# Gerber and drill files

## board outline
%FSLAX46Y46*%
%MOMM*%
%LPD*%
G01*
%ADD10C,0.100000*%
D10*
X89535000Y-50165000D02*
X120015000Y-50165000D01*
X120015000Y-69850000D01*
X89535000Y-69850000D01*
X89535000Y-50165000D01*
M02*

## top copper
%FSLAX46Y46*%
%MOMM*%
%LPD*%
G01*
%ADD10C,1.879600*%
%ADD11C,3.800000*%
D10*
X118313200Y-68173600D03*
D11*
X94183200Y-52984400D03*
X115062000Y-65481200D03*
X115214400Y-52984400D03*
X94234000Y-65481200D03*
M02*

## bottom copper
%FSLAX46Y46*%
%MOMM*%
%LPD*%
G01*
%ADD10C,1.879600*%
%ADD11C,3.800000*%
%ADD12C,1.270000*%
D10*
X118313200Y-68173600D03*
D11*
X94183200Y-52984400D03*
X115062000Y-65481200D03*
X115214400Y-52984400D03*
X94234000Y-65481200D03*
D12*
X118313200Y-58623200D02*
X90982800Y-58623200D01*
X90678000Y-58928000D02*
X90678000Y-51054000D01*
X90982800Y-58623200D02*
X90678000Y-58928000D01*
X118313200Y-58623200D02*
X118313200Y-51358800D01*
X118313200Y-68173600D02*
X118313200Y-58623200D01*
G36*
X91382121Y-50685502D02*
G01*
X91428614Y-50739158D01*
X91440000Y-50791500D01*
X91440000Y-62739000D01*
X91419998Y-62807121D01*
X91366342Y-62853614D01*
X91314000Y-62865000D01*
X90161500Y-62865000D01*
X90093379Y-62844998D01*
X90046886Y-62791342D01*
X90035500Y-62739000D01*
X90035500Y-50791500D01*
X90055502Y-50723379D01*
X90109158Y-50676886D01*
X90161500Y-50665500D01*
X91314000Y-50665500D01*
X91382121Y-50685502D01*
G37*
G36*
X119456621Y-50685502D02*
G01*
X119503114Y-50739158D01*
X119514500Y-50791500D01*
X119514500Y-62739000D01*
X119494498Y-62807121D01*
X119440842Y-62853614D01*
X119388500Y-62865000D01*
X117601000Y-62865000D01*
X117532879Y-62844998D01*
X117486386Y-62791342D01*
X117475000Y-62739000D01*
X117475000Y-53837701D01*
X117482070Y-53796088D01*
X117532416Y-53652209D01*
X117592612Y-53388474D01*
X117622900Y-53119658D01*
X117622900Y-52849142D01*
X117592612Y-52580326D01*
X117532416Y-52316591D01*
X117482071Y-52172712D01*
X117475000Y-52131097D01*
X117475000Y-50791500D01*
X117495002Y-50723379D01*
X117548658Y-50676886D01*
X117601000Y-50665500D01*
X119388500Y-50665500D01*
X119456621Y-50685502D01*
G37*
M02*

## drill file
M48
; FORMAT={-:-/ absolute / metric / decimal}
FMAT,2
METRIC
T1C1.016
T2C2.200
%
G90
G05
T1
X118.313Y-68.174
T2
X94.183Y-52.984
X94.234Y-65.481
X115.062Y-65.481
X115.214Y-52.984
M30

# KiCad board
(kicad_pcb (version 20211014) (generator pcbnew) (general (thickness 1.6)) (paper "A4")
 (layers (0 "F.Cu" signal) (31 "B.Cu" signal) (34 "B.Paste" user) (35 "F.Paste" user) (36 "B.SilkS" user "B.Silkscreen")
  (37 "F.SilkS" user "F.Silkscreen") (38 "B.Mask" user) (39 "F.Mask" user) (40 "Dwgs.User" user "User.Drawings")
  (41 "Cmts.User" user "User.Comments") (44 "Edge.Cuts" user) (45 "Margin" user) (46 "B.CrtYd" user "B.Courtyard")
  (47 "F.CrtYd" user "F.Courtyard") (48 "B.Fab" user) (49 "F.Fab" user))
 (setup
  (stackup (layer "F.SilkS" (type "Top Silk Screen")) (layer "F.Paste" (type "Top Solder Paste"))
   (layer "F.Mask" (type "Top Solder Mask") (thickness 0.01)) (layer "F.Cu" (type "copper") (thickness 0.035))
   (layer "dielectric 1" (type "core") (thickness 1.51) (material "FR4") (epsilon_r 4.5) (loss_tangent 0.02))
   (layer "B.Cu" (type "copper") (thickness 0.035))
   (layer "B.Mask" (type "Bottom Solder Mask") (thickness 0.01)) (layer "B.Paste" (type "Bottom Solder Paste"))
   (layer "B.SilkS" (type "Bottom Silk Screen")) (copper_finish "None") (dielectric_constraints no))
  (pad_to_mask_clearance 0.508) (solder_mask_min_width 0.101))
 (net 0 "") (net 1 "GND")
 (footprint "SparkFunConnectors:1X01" (layer "F.Cu") (at 118.3132 68.1736)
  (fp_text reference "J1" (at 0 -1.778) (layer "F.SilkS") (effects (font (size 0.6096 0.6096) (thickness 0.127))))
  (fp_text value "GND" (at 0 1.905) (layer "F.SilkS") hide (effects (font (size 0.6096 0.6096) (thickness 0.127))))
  (pad "1" thru_hole circle locked (at 0 0) (size 1.8796 1.8796) (drill 1.016) (layers *.Cu *.Mask) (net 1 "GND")
   (solder_mask_margin 0.1016)))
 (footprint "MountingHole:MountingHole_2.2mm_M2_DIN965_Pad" (layer "F.Cu") (at 94.1832 52.9844)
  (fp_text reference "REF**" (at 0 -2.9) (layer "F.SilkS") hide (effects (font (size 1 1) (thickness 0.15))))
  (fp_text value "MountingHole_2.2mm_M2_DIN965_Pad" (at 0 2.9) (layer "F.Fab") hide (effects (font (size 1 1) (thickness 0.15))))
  (pad "1" thru_hole circle (at 0 0) (size 3.8 3.8) (drill 2.2) (layers *.Cu *.Mask)))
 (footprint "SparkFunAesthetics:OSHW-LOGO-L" (layer "F.Cu") (at 104.775 60.325)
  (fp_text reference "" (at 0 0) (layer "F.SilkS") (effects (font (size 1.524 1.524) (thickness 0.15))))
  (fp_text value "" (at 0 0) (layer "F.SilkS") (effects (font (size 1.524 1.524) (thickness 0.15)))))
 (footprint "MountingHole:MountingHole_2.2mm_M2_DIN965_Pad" (layer "F.Cu") (at 115.062 65.4812)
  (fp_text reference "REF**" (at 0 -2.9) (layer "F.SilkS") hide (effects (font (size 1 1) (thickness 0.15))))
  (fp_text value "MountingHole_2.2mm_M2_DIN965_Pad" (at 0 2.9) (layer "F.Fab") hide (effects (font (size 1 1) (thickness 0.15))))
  (pad "1" thru_hole circle (at 0 0) (size 3.8 3.8) (drill 2.2) (layers *.Cu *.Mask)))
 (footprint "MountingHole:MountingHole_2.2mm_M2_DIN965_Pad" (layer "F.Cu") (at 115.2144 52.9844)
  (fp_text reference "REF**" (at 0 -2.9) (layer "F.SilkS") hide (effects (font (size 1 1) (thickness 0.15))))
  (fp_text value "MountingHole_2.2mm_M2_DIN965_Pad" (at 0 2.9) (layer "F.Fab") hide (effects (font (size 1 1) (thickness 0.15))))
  (pad "1" thru_hole circle (at 0 0) (size 3.8 3.8) (drill 2.2) (layers *.Cu *.Mask)))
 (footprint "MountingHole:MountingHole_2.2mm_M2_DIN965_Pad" (layer "F.Cu") (at 94.234 65.4812)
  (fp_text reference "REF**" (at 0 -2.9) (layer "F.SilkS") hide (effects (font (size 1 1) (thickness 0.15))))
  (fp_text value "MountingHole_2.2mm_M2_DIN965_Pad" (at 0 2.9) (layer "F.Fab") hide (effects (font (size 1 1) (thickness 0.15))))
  (pad "1" thru_hole circle (at 0 0) (size 3.8 3.8) (drill 2.2) (layers *.Cu *.Mask)))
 (gr_rect (start 120.015 50.165) (end 89.535 69.85) (layer "Edge.Cuts") (width 0.1) (fill none))
 (segment (start 118.3132 58.6232) (end 90.9828 58.6232) (width 1.27) (layer "B.Cu") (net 1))
 (segment (start 90.678 58.928) (end 90.678 51.054) (width 1.27) (layer "B.Cu") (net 1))
 (segment (start 90.9828 58.6232) (end 90.678 58.928) (width 1.27) (layer "B.Cu") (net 1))
 (segment (start 118.3132 58.6232) (end 118.3132 51.3588) (width 1.27) (layer "B.Cu") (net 1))
 (segment (start 118.3132 68.1736) (end 118.3132 58.6232) (width 1.27) (layer "B.Cu") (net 1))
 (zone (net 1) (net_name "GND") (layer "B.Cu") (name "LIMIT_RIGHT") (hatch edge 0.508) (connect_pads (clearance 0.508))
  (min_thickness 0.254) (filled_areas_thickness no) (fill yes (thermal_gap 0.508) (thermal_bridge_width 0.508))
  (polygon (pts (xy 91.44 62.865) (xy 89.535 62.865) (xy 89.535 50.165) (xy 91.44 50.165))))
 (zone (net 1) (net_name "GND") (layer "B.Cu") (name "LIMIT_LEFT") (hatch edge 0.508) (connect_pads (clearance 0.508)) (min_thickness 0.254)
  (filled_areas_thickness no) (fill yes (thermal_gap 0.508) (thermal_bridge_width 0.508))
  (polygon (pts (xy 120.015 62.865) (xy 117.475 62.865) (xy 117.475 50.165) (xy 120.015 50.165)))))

